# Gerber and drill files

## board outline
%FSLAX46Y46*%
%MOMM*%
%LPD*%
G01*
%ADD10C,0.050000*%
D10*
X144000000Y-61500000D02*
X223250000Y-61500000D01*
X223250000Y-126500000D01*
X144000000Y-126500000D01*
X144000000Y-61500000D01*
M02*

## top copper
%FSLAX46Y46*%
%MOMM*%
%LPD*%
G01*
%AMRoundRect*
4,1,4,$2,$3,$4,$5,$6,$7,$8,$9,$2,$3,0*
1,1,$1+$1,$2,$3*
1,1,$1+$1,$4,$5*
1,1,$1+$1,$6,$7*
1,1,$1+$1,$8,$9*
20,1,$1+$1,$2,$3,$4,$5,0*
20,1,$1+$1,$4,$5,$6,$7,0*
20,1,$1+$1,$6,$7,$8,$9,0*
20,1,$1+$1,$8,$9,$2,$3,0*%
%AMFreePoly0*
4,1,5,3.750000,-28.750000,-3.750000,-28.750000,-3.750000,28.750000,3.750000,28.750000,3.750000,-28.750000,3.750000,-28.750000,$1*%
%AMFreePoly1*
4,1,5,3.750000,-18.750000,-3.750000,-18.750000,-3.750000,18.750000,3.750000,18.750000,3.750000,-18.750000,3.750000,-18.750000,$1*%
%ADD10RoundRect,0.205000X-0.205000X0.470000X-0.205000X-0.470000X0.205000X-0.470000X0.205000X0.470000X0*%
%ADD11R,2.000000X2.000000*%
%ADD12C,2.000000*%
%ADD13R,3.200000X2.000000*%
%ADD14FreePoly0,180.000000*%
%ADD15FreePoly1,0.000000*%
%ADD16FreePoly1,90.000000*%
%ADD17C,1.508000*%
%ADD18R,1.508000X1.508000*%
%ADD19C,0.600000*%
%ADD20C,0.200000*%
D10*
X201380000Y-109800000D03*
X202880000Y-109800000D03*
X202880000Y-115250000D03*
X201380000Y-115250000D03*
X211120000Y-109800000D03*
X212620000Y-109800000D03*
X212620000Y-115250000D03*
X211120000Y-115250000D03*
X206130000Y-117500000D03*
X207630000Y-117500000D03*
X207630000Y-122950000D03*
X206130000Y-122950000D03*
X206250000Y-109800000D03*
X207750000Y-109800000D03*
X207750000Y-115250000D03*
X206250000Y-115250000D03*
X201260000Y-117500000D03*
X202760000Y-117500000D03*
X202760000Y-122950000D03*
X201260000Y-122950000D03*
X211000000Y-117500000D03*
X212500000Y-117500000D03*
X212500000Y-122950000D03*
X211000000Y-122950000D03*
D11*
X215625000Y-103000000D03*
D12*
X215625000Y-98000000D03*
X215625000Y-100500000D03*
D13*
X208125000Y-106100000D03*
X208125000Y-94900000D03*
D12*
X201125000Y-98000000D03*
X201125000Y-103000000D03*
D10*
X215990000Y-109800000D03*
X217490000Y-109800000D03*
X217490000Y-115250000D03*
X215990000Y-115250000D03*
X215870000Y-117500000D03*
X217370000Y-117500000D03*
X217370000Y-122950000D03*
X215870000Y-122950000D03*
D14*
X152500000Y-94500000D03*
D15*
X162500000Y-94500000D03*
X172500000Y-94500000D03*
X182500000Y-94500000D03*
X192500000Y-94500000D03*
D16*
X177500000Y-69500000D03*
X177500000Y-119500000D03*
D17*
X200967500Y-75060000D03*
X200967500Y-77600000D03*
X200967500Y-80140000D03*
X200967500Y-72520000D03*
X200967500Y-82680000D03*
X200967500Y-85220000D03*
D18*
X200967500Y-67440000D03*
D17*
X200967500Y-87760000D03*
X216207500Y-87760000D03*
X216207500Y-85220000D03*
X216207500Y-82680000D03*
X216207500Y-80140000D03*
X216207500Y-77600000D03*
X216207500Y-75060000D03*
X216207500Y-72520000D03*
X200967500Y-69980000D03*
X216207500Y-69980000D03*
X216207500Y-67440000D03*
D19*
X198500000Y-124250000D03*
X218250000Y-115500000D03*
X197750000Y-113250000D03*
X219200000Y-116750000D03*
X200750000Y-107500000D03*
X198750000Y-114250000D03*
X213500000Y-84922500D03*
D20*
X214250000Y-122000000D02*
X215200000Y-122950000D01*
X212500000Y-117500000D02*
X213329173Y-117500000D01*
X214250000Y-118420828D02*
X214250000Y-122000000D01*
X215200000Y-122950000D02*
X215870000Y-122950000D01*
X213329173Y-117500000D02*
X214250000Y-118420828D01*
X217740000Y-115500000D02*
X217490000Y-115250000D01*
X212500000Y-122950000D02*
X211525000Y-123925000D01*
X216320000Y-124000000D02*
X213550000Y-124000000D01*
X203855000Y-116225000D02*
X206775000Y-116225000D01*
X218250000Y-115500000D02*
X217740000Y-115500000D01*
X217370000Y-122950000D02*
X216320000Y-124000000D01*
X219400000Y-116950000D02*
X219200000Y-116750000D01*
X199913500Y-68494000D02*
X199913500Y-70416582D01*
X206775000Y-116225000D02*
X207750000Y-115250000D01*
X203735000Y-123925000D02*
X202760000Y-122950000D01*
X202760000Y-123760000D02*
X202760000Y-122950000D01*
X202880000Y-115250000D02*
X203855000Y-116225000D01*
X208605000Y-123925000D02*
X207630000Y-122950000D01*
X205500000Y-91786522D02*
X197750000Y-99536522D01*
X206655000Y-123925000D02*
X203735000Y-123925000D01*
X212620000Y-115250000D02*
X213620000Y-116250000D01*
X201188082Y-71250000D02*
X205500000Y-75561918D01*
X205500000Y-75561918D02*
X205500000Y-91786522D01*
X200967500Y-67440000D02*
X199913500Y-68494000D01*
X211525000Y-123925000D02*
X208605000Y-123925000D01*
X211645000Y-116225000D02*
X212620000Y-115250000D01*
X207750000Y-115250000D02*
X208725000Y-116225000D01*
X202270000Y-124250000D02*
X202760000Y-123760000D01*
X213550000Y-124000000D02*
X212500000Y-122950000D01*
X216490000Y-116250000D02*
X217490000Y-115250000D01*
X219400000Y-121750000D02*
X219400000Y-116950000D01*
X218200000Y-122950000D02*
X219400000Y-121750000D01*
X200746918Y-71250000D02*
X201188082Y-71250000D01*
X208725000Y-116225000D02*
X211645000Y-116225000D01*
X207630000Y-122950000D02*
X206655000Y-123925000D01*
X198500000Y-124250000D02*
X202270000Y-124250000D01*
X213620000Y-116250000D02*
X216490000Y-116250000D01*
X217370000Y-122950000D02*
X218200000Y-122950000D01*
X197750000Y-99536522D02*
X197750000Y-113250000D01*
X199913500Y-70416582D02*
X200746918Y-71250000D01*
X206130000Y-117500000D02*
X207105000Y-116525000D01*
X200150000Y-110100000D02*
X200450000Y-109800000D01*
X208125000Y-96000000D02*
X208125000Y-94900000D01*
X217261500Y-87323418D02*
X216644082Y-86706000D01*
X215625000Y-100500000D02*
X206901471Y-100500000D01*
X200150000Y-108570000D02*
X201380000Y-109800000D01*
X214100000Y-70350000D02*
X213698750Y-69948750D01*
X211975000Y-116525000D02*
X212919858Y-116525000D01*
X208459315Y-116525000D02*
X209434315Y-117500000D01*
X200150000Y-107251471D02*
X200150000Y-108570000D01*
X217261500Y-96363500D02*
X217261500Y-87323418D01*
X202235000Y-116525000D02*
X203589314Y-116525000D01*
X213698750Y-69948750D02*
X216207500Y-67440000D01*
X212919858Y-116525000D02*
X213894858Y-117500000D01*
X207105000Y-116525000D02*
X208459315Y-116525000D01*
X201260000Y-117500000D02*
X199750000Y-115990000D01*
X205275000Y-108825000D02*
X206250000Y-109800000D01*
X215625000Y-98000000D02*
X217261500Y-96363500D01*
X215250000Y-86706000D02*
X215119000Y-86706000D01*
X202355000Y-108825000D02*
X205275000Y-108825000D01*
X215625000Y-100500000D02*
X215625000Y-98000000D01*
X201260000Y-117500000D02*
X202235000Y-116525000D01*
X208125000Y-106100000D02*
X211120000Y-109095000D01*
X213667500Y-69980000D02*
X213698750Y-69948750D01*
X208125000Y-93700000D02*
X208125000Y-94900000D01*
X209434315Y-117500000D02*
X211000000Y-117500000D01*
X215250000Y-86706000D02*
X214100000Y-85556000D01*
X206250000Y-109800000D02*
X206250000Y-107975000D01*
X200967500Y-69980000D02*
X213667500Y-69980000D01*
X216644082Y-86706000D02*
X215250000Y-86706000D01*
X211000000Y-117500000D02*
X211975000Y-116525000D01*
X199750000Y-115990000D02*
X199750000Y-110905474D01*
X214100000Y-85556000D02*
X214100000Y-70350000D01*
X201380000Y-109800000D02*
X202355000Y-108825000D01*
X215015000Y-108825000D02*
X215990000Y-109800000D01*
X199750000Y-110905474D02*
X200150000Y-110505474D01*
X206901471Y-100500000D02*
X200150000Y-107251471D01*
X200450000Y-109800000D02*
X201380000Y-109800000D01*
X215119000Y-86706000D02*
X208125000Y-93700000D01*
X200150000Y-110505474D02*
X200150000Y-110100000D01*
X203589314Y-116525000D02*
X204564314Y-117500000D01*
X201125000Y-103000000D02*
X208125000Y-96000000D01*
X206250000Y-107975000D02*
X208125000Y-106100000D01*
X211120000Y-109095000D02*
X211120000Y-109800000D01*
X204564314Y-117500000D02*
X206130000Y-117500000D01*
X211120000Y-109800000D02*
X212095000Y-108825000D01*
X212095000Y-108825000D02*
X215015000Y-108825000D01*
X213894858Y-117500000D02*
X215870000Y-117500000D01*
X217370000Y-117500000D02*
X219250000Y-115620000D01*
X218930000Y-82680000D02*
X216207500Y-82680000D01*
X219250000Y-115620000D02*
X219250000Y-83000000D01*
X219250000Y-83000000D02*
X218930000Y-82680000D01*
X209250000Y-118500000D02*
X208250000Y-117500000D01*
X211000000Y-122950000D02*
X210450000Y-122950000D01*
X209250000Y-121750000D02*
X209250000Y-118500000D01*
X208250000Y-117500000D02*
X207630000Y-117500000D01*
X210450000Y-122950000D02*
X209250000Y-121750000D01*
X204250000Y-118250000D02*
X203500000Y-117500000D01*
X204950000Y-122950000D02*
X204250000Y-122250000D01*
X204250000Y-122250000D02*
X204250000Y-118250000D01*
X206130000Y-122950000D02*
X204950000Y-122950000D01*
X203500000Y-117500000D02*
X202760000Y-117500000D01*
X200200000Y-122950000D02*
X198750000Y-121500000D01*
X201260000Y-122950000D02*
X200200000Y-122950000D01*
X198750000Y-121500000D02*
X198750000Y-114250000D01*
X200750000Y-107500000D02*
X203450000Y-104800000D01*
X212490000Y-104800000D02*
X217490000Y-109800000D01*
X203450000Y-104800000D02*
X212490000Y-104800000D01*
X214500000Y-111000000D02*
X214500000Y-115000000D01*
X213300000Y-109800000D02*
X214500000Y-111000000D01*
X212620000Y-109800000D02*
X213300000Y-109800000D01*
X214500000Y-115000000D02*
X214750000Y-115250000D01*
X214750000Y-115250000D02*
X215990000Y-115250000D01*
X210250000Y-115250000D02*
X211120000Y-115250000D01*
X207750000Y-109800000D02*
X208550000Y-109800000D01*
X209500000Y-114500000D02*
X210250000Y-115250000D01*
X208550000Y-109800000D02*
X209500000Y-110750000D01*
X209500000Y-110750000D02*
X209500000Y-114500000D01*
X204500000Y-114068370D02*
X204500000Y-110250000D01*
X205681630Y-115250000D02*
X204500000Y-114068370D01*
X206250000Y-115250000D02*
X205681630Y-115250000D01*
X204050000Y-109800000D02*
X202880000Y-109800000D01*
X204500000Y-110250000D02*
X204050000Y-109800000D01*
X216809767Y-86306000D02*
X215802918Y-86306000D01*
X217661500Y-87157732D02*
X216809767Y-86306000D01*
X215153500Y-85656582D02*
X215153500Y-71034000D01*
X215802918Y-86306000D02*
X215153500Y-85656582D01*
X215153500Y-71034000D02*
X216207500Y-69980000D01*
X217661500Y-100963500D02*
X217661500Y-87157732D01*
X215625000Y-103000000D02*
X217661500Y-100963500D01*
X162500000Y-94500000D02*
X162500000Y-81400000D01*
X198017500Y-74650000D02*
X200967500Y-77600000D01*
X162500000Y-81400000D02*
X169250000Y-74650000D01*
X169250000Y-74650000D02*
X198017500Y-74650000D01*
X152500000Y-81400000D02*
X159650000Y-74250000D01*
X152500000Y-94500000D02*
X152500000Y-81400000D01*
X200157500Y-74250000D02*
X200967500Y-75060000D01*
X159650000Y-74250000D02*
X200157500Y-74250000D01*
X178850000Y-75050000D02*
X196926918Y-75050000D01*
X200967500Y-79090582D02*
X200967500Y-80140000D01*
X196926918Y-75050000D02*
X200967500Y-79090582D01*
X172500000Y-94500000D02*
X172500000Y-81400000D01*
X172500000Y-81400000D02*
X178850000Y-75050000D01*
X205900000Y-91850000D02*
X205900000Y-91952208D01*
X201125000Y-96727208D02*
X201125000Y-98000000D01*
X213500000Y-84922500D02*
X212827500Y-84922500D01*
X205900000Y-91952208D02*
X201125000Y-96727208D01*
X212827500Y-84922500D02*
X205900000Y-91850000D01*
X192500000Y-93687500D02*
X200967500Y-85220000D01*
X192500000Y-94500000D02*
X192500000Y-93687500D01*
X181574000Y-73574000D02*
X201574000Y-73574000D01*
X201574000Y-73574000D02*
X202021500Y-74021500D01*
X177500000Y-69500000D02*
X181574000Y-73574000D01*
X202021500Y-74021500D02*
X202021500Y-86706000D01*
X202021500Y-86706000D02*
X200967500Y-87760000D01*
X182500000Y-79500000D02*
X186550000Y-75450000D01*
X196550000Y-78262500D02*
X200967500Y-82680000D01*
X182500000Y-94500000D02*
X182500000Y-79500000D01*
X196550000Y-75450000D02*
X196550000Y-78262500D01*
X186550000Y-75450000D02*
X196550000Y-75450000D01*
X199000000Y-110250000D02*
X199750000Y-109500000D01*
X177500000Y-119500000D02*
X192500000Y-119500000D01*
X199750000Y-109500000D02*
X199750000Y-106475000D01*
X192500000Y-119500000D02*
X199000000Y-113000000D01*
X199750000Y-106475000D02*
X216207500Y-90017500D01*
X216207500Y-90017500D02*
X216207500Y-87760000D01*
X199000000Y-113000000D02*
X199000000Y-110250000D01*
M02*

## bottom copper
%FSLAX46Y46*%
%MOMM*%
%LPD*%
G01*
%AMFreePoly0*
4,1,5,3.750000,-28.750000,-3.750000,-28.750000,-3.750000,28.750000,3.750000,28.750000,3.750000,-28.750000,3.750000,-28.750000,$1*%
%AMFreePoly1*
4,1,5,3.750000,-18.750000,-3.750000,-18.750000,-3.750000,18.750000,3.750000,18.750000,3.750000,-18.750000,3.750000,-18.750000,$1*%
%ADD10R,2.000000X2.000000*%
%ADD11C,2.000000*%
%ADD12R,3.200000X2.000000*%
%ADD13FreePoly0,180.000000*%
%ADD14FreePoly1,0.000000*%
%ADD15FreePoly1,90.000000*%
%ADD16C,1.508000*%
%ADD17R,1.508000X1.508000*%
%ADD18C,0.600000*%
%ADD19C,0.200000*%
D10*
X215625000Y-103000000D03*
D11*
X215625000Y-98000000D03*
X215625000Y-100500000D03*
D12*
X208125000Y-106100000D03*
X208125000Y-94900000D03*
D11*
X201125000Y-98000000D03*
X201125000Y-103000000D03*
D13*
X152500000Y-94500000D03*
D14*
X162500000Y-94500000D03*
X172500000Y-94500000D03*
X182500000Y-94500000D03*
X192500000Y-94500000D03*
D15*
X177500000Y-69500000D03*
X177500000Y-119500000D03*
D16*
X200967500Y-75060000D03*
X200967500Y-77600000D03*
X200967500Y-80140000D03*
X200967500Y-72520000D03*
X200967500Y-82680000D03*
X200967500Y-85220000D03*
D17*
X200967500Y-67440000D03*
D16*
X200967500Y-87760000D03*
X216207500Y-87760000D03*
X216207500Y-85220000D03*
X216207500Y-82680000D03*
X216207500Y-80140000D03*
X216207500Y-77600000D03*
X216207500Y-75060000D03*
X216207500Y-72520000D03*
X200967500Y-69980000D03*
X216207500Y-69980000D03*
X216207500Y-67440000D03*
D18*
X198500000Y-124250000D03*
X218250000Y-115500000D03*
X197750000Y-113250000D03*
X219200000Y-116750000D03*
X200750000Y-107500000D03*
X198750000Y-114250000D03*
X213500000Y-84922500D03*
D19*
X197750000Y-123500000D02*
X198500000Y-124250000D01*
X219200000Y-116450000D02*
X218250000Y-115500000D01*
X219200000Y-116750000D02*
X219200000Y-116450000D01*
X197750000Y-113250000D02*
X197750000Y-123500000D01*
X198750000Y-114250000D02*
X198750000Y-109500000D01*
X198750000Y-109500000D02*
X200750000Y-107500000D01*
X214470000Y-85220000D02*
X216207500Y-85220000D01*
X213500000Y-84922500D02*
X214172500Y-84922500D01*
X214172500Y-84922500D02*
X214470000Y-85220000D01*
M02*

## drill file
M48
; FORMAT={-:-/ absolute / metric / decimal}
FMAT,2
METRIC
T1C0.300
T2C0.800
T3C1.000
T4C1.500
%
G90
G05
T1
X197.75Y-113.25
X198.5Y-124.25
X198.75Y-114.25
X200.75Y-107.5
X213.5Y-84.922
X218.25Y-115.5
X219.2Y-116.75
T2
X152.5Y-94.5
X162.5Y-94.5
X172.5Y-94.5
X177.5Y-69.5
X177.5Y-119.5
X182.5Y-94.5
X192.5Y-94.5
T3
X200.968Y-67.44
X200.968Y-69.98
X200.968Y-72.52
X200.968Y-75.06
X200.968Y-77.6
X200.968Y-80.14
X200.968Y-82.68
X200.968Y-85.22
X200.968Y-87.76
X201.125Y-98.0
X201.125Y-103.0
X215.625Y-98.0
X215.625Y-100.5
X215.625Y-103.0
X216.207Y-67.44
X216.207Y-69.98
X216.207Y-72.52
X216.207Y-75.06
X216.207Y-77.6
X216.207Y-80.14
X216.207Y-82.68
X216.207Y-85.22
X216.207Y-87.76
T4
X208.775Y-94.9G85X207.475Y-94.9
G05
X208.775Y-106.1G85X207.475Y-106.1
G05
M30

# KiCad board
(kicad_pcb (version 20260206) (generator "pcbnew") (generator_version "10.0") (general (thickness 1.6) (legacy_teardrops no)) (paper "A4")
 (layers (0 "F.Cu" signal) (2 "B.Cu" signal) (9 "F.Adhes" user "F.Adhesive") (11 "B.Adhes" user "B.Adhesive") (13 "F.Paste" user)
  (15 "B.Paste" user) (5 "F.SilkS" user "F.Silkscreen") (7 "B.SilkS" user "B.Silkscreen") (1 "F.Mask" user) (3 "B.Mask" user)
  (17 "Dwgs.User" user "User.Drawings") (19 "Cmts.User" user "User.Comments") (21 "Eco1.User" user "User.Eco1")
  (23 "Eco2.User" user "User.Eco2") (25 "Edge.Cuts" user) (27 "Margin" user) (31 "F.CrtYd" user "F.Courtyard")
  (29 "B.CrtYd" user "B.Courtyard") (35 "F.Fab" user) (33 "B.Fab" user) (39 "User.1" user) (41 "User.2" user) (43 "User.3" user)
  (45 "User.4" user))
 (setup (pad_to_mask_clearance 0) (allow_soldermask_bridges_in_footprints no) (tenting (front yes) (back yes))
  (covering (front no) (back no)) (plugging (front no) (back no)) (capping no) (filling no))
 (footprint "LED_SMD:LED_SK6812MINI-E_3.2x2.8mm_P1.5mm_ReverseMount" (layer "F.Cu") (at 202.13 112.525 -90)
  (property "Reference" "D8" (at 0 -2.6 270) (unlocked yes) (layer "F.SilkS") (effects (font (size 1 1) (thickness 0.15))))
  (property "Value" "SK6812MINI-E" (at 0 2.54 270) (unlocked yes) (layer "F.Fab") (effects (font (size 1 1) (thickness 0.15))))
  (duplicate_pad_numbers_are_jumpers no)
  (pad "1" smd roundrect (at -2.725 0.75 270) (size 1.35 0.82) (layers "F.Cu" "F.Mask" "F.Paste") (roundrect_rratio 0.25) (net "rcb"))
  (pad "2" smd roundrect (at -2.725 -0.75 270) (size 1.35 0.82) (layers "F.Cu" "F.Mask" "F.Paste") (roundrect_rratio 0.25)
   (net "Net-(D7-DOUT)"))
  (pad "3" smd roundrect (at 2.725 -0.75 270) (size 1.35 0.82) (layers "F.Cu" "F.Mask" "F.Paste") (roundrect_rratio 0.25) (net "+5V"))
  (pad "4" smd roundrect (at 2.725 0.75 270) (size 1.35 0.82) (layers "F.Cu" "F.Mask" "F.Paste") (roundrect_rratio 0.25)
   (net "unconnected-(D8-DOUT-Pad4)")))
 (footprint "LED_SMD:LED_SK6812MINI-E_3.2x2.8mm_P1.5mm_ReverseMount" (layer "F.Cu") (at 211.87 112.525 -90)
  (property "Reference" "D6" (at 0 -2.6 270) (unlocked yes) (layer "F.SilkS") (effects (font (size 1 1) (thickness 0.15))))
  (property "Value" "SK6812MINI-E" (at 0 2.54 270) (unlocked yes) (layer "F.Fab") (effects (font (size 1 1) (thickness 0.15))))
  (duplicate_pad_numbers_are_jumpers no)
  (pad "1" smd roundrect (at -2.725 0.75 270) (size 1.35 0.82) (layers "F.Cu" "F.Mask" "F.Paste") (roundrect_rratio 0.25) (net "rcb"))
  (pad "2" smd roundrect (at -2.725 -0.75 270) (size 1.35 0.82) (layers "F.Cu" "F.Mask" "F.Paste") (roundrect_rratio 0.25)
   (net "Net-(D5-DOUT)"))
  (pad "3" smd roundrect (at 2.725 -0.75 270) (size 1.35 0.82) (layers "F.Cu" "F.Mask" "F.Paste") (roundrect_rratio 0.25) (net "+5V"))
  (pad "4" smd roundrect (at 2.725 0.75 270) (size 1.35 0.82) (layers "F.Cu" "F.Mask" "F.Paste") (roundrect_rratio 0.25)
   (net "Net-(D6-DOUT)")))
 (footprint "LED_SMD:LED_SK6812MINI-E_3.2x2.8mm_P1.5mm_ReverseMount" (layer "F.Cu") (at 206.88 120.225 -90)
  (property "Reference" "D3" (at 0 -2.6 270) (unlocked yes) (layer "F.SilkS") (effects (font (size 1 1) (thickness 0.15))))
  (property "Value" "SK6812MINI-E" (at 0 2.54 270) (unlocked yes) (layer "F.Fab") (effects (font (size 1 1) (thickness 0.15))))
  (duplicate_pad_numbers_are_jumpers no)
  (pad "1" smd roundrect (at -2.725 0.75 270) (size 1.35 0.82) (layers "F.Cu" "F.Mask" "F.Paste") (roundrect_rratio 0.25) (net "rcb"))
  (pad "2" smd roundrect (at -2.725 -0.75 270) (size 1.35 0.82) (layers "F.Cu" "F.Mask" "F.Paste") (roundrect_rratio 0.25)
   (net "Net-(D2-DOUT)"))
  (pad "3" smd roundrect (at 2.725 -0.75 270) (size 1.35 0.82) (layers "F.Cu" "F.Mask" "F.Paste") (roundrect_rratio 0.25) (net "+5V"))
  (pad "4" smd roundrect (at 2.725 0.75 270) (size 1.35 0.82) (layers "F.Cu" "F.Mask" "F.Paste") (roundrect_rratio 0.25)
   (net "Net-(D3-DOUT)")))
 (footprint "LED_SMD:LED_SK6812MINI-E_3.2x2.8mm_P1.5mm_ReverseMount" (layer "F.Cu") (at 207 112.525 -90)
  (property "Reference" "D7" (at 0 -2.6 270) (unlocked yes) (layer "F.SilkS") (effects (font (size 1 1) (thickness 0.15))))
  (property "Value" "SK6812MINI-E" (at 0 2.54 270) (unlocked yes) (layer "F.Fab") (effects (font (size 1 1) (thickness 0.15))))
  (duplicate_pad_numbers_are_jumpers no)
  (pad "1" smd roundrect (at -2.725 0.75 270) (size 1.35 0.82) (layers "F.Cu" "F.Mask" "F.Paste") (roundrect_rratio 0.25) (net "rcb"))
  (pad "2" smd roundrect (at -2.725 -0.75 270) (size 1.35 0.82) (layers "F.Cu" "F.Mask" "F.Paste") (roundrect_rratio 0.25)
   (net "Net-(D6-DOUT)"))
  (pad "3" smd roundrect (at 2.725 -0.75 270) (size 1.35 0.82) (layers "F.Cu" "F.Mask" "F.Paste") (roundrect_rratio 0.25) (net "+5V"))
  (pad "4" smd roundrect (at 2.725 0.75 270) (size 1.35 0.82) (layers "F.Cu" "F.Mask" "F.Paste") (roundrect_rratio 0.25)
   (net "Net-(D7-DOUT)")))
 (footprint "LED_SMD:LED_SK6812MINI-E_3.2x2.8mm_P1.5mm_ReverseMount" (layer "F.Cu") (at 202.01 120.225 -90)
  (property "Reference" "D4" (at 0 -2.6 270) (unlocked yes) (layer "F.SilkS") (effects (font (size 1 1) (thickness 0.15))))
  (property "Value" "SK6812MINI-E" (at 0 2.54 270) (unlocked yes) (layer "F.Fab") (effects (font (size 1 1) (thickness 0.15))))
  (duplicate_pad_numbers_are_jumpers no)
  (pad "1" smd roundrect (at -2.725 0.75 270) (size 1.35 0.82) (layers "F.Cu" "F.Mask" "F.Paste") (roundrect_rratio 0.25) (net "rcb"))
  (pad "2" smd roundrect (at -2.725 -0.75 270) (size 1.35 0.82) (layers "F.Cu" "F.Mask" "F.Paste") (roundrect_rratio 0.25)
   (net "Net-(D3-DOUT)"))
  (pad "3" smd roundrect (at 2.725 -0.75 270) (size 1.35 0.82) (layers "F.Cu" "F.Mask" "F.Paste") (roundrect_rratio 0.25) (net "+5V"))
  (pad "4" smd roundrect (at 2.725 0.75 270) (size 1.35 0.82) (layers "F.Cu" "F.Mask" "F.Paste") (roundrect_rratio 0.25)
   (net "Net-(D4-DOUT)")))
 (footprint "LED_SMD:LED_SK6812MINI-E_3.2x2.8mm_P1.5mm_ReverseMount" (layer "F.Cu") (at 211.75 120.225 -90)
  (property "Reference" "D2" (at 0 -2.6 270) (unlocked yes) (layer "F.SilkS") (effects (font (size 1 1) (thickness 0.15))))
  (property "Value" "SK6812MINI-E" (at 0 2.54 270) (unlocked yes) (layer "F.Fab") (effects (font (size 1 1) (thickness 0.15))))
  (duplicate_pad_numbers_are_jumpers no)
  (pad "1" smd roundrect (at -2.725 0.75 270) (size 1.35 0.82) (layers "F.Cu" "F.Mask" "F.Paste") (roundrect_rratio 0.25) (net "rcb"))
  (pad "2" smd roundrect (at -2.725 -0.75 270) (size 1.35 0.82) (layers "F.Cu" "F.Mask" "F.Paste") (roundrect_rratio 0.25)
   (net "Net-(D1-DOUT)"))
  (pad "3" smd roundrect (at 2.725 -0.75 270) (size 1.35 0.82) (layers "F.Cu" "F.Mask" "F.Paste") (roundrect_rratio 0.25) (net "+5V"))
  (pad "4" smd roundrect (at 2.725 0.75 270) (size 1.35 0.82) (layers "F.Cu" "F.Mask" "F.Paste") (roundrect_rratio 0.25)
   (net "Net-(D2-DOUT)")))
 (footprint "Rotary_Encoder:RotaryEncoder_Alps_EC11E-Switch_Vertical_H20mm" (layer "F.Cu") (at 215.625 103 180)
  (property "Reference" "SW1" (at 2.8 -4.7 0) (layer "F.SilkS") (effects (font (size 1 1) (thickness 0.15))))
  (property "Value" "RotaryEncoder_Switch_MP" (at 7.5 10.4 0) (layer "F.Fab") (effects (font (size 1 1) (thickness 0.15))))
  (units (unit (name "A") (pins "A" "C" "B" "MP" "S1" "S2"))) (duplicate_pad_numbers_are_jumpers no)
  (pad "A" thru_hole rect (at 0 0 180) (size 2 2) (drill 1) (layers "*.Cu" "*.Mask") (remove_unused_layers no) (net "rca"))
  (pad "B" thru_hole circle (at 0 5 180) (size 2 2) (drill 1) (layers "*.Cu" "*.Mask") (remove_unused_layers no) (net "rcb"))
  (pad "C" thru_hole circle (at 0 2.5 180) (size 2 2) (drill 1) (layers "*.Cu" "*.Mask") (remove_unused_layers no) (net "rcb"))
  (pad "MP" thru_hole rect (at 7.5 -3.1 180) (size 3.2 2) (drill oval 2.8 1.5) (layers "*.Cu" "*.Mask") (remove_unused_layers no)
   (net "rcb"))
  (pad "MP" thru_hole rect (at 7.5 8.1 180) (size 3.2 2) (drill oval 2.8 1.5) (layers "*.Cu" "*.Mask") (remove_unused_layers no) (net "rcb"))
  (pad "S1" thru_hole circle (at 14.5 5 180) (size 2 2) (drill 1) (layers "*.Cu" "*.Mask") (remove_unused_layers no) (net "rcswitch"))
  (pad "S2" thru_hole circle (at 14.5 0 180) (size 2 2) (drill 1) (layers "*.Cu" "*.Mask") (remove_unused_layers no) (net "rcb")))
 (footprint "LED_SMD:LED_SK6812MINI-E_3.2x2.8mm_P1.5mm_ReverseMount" (layer "F.Cu") (at 216.74 112.525 -90)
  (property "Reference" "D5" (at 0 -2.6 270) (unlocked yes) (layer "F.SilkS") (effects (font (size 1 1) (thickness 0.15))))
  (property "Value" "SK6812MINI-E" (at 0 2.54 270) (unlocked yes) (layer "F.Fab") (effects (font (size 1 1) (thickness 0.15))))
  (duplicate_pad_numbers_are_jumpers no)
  (pad "1" smd roundrect (at -2.725 0.75 270) (size 1.35 0.82) (layers "F.Cu" "F.Mask" "F.Paste") (roundrect_rratio 0.25) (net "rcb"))
  (pad "2" smd roundrect (at -2.725 -0.75 270) (size 1.35 0.82) (layers "F.Cu" "F.Mask" "F.Paste") (roundrect_rratio 0.25)
   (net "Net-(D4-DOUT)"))
  (pad "3" smd roundrect (at 2.725 -0.75 270) (size 1.35 0.82) (layers "F.Cu" "F.Mask" "F.Paste") (roundrect_rratio 0.25) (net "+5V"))
  (pad "4" smd roundrect (at 2.725 0.75 270) (size 1.35 0.82) (layers "F.Cu" "F.Mask" "F.Paste") (roundrect_rratio 0.25)
   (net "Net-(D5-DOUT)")))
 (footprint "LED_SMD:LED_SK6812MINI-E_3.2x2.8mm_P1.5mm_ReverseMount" (layer "F.Cu") (at 216.62 120.225 -90)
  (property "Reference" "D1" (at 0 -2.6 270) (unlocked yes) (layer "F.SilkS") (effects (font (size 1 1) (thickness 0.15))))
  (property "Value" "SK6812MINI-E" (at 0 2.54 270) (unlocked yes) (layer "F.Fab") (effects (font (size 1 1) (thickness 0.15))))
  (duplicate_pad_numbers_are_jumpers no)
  (pad "1" smd roundrect (at -2.725 0.75 270) (size 1.35 0.82) (layers "F.Cu" "F.Mask" "F.Paste") (roundrect_rratio 0.25) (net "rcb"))
  (pad "2" smd roundrect (at -2.725 -0.75 270) (size 1.35 0.82) (layers "F.Cu" "F.Mask" "F.Paste") (roundrect_rratio 0.25) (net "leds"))
  (pad "3" smd roundrect (at 2.725 -0.75 270) (size 1.35 0.82) (layers "F.Cu" "F.Mask" "F.Paste") (roundrect_rratio 0.25) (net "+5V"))
  (pad "4" smd roundrect (at 2.725 0.75 270) (size 1.35 0.82) (layers "F.Cu" "F.Mask" "F.Paste") (roundrect_rratio 0.25)
   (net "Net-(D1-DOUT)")))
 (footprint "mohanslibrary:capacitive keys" (layer "F.Cu") (at 179.5 94.5 -90)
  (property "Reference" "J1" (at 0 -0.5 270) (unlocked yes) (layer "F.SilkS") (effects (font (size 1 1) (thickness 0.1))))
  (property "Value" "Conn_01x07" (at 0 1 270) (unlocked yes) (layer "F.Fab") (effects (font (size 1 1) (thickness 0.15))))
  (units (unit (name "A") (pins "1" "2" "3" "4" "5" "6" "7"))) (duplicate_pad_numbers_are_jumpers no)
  (pad "1" thru_hole custom (at 0 27 180) (size 7.5 57.5) (drill 0.8) (layers "*.Cu" "*.Mask") (remove_unused_layers no) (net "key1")
   (options (clearance outline) (anchor rect)) (primitives))
  (pad "2" thru_hole custom (at 0 17) (size 7.5 37.5) (drill 0.8) (layers "*.Cu" "*.Mask") (remove_unused_layers no) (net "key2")
   (options (clearance outline) (anchor rect)) (primitives))
  (pad "3" thru_hole custom (at 0 7) (size 7.5 37.5) (drill 0.8) (layers "*.Cu" "*.Mask") (remove_unused_layers no) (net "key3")
   (options (clearance outline) (anchor rect)) (primitives))
  (pad "4" thru_hole custom (at 0 -3) (size 7.5 37.5) (drill 0.8) (layers "*.Cu" "*.Mask") (remove_unused_layers no) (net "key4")
   (options (clearance outline) (anchor rect)) (primitives))
  (pad "5" thru_hole custom (at 0 -13) (size 7.5 37.5) (drill 0.8) (layers "*.Cu" "*.Mask") (remove_unused_layers no) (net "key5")
   (options (clearance outline) (anchor rect)) (primitives))
  (pad "6" thru_hole custom (at -25 2 90) (size 7.5 37.5) (drill 0.8) (layers "*.Cu" "*.Mask") (remove_unused_layers no) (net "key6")
   (options (clearance outline) (anchor rect)) (primitives))
  (pad "7" thru_hole custom (at 25 2 90) (size 7.5 37.5) (drill 0.8) (layers "*.Cu" "*.Mask") (remove_unused_layers no) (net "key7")
   (options (clearance outline) (anchor rect)) (primitives)))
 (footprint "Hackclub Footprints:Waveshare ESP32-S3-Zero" (layer "F.Cu") (at 208.5875 77.6)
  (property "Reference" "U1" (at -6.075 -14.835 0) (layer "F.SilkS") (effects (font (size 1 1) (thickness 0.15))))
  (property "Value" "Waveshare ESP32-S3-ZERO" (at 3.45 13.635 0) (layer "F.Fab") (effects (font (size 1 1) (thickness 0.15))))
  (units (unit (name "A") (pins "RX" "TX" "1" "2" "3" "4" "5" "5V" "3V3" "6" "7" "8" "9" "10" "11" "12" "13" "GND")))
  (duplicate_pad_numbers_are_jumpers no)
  (pad "1" thru_hole circle (at -7.62 -2.54) (size 1.508 1.508) (drill 1) (layers "*.Cu" "*.Mask") (remove_unused_layers no) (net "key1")
   (solder_mask_margin 0.102))
  (pad "2" thru_hole circle (at -7.62 0) (size 1.508 1.508) (drill 1) (layers "*.Cu" "*.Mask") (remove_unused_layers no) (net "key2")
   (solder_mask_margin 0.102))
  (pad "3" thru_hole circle (at -7.62 2.54) (size 1.508 1.508) (drill 1) (layers "*.Cu" "*.Mask") (remove_unused_layers no) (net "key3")
   (solder_mask_margin 0.102))
  (pad "3V3" thru_hole circle (at -7.62 -5.08) (size 1.508 1.508) (drill 1) (layers "*.Cu" "*.Mask") (remove_unused_layers no) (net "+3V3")
   (solder_mask_margin 0.102))
  (pad "4" thru_hole circle (at -7.62 5.08) (size 1.508 1.508) (drill 1) (layers "*.Cu" "*.Mask") (remove_unused_layers no) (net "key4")
   (solder_mask_margin 0.102))
  (pad "5" thru_hole circle (at -7.62 7.62) (size 1.508 1.508) (drill 1) (layers "*.Cu" "*.Mask") (remove_unused_layers no) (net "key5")
   (solder_mask_margin 0.102))
  (pad "5V" thru_hole rect (at -7.62 -10.16) (size 1.508 1.508) (drill 1) (layers "*.Cu" "*.Mask") (remove_unused_layers no) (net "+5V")
   (solder_mask_margin 0.102))
  (pad "6" thru_hole circle (at -7.62 10.16) (size 1.508 1.508) (drill 1) (layers "*.Cu" "*.Mask") (remove_unused_layers no) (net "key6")
   (solder_mask_margin 0.102))
  (pad "7" thru_hole circle (at 7.62 10.16) (size 1.508 1.508) (drill 1) (layers "*.Cu" "*.Mask") (remove_unused_layers no) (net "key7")
   (solder_mask_margin 0.102))
  (pad "8" thru_hole circle (at 7.62 7.62) (size 1.508 1.508) (drill 1) (layers "*.Cu" "*.Mask") (remove_unused_layers no) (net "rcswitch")
   (solder_mask_margin 0.102))
  (pad "9" thru_hole circle (at 7.62 5.08) (size 1.508 1.508) (drill 1) (layers "*.Cu" "*.Mask") (remove_unused_layers no) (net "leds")
   (solder_mask_margin 0.102))
  (pad "10" thru_hole circle (at 7.62 2.54) (size 1.508 1.508) (drill 1) (layers "*.Cu" "*.Mask") (remove_unused_layers no)
   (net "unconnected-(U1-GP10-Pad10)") (solder_mask_margin 0.102))
  (pad "11" thru_hole circle (at 7.62 0) (size 1.508 1.508) (drill 1) (layers "*.Cu" "*.Mask") (remove_unused_layers no)
   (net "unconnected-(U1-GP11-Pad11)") (solder_mask_margin 0.102))
  (pad "12" thru_hole circle (at 7.62 -2.54) (size 1.508 1.508) (drill 1) (layers "*.Cu" "*.Mask") (remove_unused_layers no)
   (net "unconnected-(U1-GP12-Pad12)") (solder_mask_margin 0.102))
  (pad "13" thru_hole circle (at 7.62 -5.08) (size 1.508 1.508) (drill 1) (layers "*.Cu" "*.Mask") (remove_unused_layers no)
   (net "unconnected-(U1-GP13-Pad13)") (solder_mask_margin 0.102))
  (pad "GND" thru_hole circle (at -7.62 -7.62) (size 1.508 1.508) (drill 1) (layers "*.Cu" "*.Mask") (remove_unused_layers no) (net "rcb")
   (solder_mask_margin 0.102))
  (pad "RX" thru_hole circle (at 7.62 -7.62) (size 1.508 1.508) (drill 1) (layers "*.Cu" "*.Mask") (remove_unused_layers no) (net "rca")
   (solder_mask_margin 0.102))
  (pad "TX" thru_hole circle (at 7.62 -10.16) (size 1.508 1.508) (drill 1) (layers "*.Cu" "*.Mask") (remove_unused_layers no) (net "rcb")
   (solder_mask_margin 0.102)))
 (gr_rect (start 144 61.5) (end 223.25 126.5) (stroke (width 0.05) (type default)) (fill no) (layer "Edge.Cuts"))
 (segment (start 214.25 122) (end 215.2 122.95) (width 0.2) (layer "F.Cu") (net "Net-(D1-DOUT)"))
 (segment (start 212.5 117.5) (end 213.329173 117.5) (width 0.2) (layer "F.Cu") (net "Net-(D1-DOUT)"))
 (segment (start 214.25 118.420828) (end 214.25 122) (width 0.2) (layer "F.Cu") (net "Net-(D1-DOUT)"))
 (segment (start 215.2 122.95) (end 215.87 122.95) (width 0.2) (layer "F.Cu") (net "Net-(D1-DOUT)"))
 (segment (start 213.329173 117.5) (end 214.25 118.420828) (width 0.2) (layer "F.Cu") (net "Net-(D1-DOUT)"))
 (segment (start 217.74 115.5) (end 217.49 115.25) (width 0.2) (layer "F.Cu") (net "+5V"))
 (segment (start 212.5 122.95) (end 211.525 123.925) (width 0.2) (layer "F.Cu") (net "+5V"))
 (segment (start 216.32 124) (end 213.55 124) (width 0.2) (layer "F.Cu") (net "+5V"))
 (segment (start 203.855 116.225) (end 206.775 116.225) (width 0.2) (layer "F.Cu") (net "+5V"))
 (segment (start 218.25 115.5) (end 217.74 115.5) (width 0.2) (layer "F.Cu") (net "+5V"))
 (segment (start 217.37 122.95) (end 216.32 124) (width 0.2) (layer "F.Cu") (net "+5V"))
 (segment (start 219.4 116.95) (end 219.2 116.75) (width 0.2) (layer "F.Cu") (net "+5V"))
 (segment (start 199.9135 68.494) (end 199.9135 70.416582) (width 0.2) (layer "F.Cu") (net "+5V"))
 (segment (start 206.775 116.225) (end 207.75 115.25) (width 0.2) (layer "F.Cu") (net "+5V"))
 (segment (start 203.735 123.925) (end 202.76 122.95) (width 0.2) (layer "F.Cu") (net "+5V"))
 (segment (start 202.76 123.76) (end 202.76 122.95) (width 0.2) (layer "F.Cu") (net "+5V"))
 (segment (start 202.88 115.25) (end 203.855 116.225) (width 0.2) (layer "F.Cu") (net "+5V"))
 (segment (start 208.605 123.925) (end 207.63 122.95) (width 0.2) (layer "F.Cu") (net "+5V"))
 (segment (start 205.5 91.786522) (end 197.75 99.536522) (width 0.2) (layer "F.Cu") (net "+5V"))
 (segment (start 206.655 123.925) (end 203.735 123.925) (width 0.2) (layer "F.Cu") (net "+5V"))
 (segment (start 212.62 115.25) (end 213.62 116.25) (width 0.2) (layer "F.Cu") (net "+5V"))
 (segment (start 201.188082 71.25) (end 205.5 75.561918) (width 0.2) (layer "F.Cu") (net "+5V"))
 (segment (start 205.5 75.561918) (end 205.5 91.786522) (width 0.2) (layer "F.Cu") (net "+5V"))
 (segment (start 200.9675 67.44) (end 199.9135 68.494) (width 0.2) (layer "F.Cu") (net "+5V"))
 (segment (start 211.525 123.925) (end 208.605 123.925) (width 0.2) (layer "F.Cu") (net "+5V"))
 (segment (start 211.645 116.225) (end 212.62 115.25) (width 0.2) (layer "F.Cu") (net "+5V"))
 (segment (start 207.75 115.25) (end 208.725 116.225) (width 0.2) (layer "F.Cu") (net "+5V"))
 (segment (start 202.27 124.25) (end 202.76 123.76) (width 0.2) (layer "F.Cu") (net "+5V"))
 (segment (start 213.55 124) (end 212.5 122.95) (width 0.2) (layer "F.Cu") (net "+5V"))
 (segment (start 216.49 116.25) (end 217.49 115.25) (width 0.2) (layer "F.Cu") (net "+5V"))
 (segment (start 219.4 121.75) (end 219.4 116.95) (width 0.2) (layer "F.Cu") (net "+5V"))
 (segment (start 218.2 122.95) (end 219.4 121.75) (width 0.2) (layer "F.Cu") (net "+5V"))
 (segment (start 200.746918 71.25) (end 201.188082 71.25) (width 0.2) (layer "F.Cu") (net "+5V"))
 (segment (start 208.725 116.225) (end 211.645 116.225) (width 0.2) (layer "F.Cu") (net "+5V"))
 (segment (start 207.63 122.95) (end 206.655 123.925) (width 0.2) (layer "F.Cu") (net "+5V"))
 (segment (start 198.5 124.25) (end 202.27 124.25) (width 0.2) (layer "F.Cu") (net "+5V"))
 (segment (start 213.62 116.25) (end 216.49 116.25) (width 0.2) (layer "F.Cu") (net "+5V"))
 (segment (start 217.37 122.95) (end 218.2 122.95) (width 0.2) (layer "F.Cu") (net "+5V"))
 (segment (start 197.75 99.536522) (end 197.75 113.25) (width 0.2) (layer "F.Cu") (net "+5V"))
 (segment (start 199.9135 70.416582) (end 200.746918 71.25) (width 0.2) (layer "F.Cu") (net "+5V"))
 (via (at 198.5 124.25) (size 0.6) (drill 0.3) (layers "F.Cu" "B.Cu") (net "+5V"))
 (via (at 218.25 115.5) (size 0.6) (drill 0.3) (layers "F.Cu" "B.Cu") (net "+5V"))
 (via (at 197.75 113.25) (size 0.6) (drill 0.3) (layers "F.Cu" "B.Cu") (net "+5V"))
 (via (at 219.2 116.75) (size 0.6) (drill 0.3) (layers "F.Cu" "B.Cu") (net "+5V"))
 (segment (start 197.75 123.5) (end 198.5 124.25) (width 0.2) (layer "B.Cu") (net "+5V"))
 (segment (start 219.2 116.45) (end 218.25 115.5) (width 0.2) (layer "B.Cu") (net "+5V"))
 (segment (start 219.2 116.75) (end 219.2 116.45) (width 0.2) (layer "B.Cu") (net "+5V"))
 (segment (start 197.75 113.25) (end 197.75 123.5) (width 0.2) (layer "B.Cu") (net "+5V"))
 (segment (start 206.13 117.5) (end 207.105 116.525) (width 0.2) (layer "F.Cu") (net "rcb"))
 (segment (start 200.15 110.1) (end 200.45 109.8) (width 0.2) (layer "F.Cu") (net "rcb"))
 (segment (start 208.125 96) (end 208.125 94.9) (width 0.2) (layer "F.Cu") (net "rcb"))
 (segment (start 217.2615 87.323418) (end 216.644082 86.706) (width 0.2) (layer "F.Cu") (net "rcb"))
 (segment (start 215.625 100.5) (end 206.901471 100.5) (width 0.2) (layer "F.Cu") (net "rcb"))
 (segment (start 200.15 108.57) (end 201.38 109.8) (width 0.2) (layer "F.Cu") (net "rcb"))
 (segment (start 214.1 70.35) (end 213.69875 69.94875) (width 0.2) (layer "F.Cu") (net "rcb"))
 (segment (start 211.975 116.525) (end 212.919858 116.525) (width 0.2) (layer "F.Cu") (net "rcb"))
 (segment (start 208.459315 116.525) (end 209.434315 117.5) (width 0.2) (layer "F.Cu") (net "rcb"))
 (segment (start 200.15 107.251471) (end 200.15 108.57) (width 0.2) (layer "F.Cu") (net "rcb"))
 (segment (start 217.2615 96.3635) (end 217.2615 87.323418) (width 0.2) (layer "F.Cu") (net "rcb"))
 (segment (start 202.235 116.525) (end 203.589314 116.525) (width 0.2) (layer "F.Cu") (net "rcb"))
 (segment (start 213.69875 69.94875) (end 216.2075 67.44) (width 0.2) (layer "F.Cu") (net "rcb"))
 (segment (start 212.919858 116.525) (end 213.894858 117.5) (width 0.2) (layer "F.Cu") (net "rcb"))
 (segment (start 207.105 116.525) (end 208.459315 116.525) (width 0.2) (layer "F.Cu") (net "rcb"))
 (segment (start 201.26 117.5) (end 199.75 115.99) (width 0.2) (layer "F.Cu") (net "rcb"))
 (segment (start 205.275 108.825) (end 206.25 109.8) (width 0.2) (layer "F.Cu") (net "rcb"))
 (segment (start 215.625 98) (end 217.2615 96.3635) (width 0.2) (layer "F.Cu") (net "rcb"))
 (segment (start 215.25 86.706) (end 215.119 86.706) (width 0.2) (layer "F.Cu") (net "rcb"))
 (segment (start 202.355 108.825) (end 205.275 108.825) (width 0.2) (layer "F.Cu") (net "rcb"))
 (segment (start 215.625 100.5) (end 215.625 98) (width 0.2) (layer "F.Cu") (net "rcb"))
 (segment (start 201.26 117.5) (end 202.235 116.525) (width 0.2) (layer "F.Cu") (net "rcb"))
 (segment (start 208.125 106.1) (end 211.12 109.095) (width 0.2) (layer "F.Cu") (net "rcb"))
 (segment (start 213.6675 69.98) (end 213.69875 69.94875) (width 0.2) (layer "F.Cu") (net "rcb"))
 (segment (start 208.125 93.7) (end 208.125 94.9) (width 0.2) (layer "F.Cu") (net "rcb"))
 (segment (start 209.434315 117.5) (end 211 117.5) (width 0.2) (layer "F.Cu") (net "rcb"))
 (segment (start 215.25 86.706) (end 214.1 85.556) (width 0.2) (layer "F.Cu") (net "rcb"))
 (segment (start 206.25 109.8) (end 206.25 107.975) (width 0.2) (layer "F.Cu") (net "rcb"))
 (segment (start 200.9675 69.98) (end 213.6675 69.98) (width 0.2) (layer "F.Cu") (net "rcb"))
 (segment (start 216.644082 86.706) (end 215.25 86.706) (width 0.2) (layer "F.Cu") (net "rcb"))
 (segment (start 211 117.5) (end 211.975 116.525) (width 0.2) (layer "F.Cu") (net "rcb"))
 (segment (start 199.75 115.99) (end 199.75 110.905474) (width 0.2) (layer "F.Cu") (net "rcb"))
 (segment (start 214.1 85.556) (end 214.1 70.35) (width 0.2) (layer "F.Cu") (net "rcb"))
 (segment (start 201.38 109.8) (end 202.355 108.825) (width 0.2) (layer "F.Cu") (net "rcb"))
 (segment (start 215.015 108.825) (end 215.99 109.8) (width 0.2) (layer "F.Cu") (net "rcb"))
 (segment (start 199.75 110.905474) (end 200.15 110.505474) (width 0.2) (layer "F.Cu") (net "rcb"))
 (segment (start 206.901471 100.5) (end 200.15 107.251471) (width 0.2) (layer "F.Cu") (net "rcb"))
 (segment (start 200.45 109.8) (end 201.38 109.8) (width 0.2) (layer "F.Cu") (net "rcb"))
 (segment (start 215.119 86.706) (end 208.125 93.7) (width 0.2) (layer "F.Cu") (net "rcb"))
 (segment (start 200.15 110.505474) (end 200.15 110.1) (width 0.2) (layer "F.Cu") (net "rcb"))
 (segment (start 203.589314 116.525) (end 204.564314 117.5) (width 0.2) (layer "F.Cu") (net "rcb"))
 (segment (start 201.125 103) (end 208.125 96) (width 0.2) (layer "F.Cu") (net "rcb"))
 (segment (start 206.25 107.975) (end 208.125 106.1) (width 0.2) (layer "F.Cu") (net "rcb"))
 (segment (start 211.12 109.095) (end 211.12 109.8) (width 0.2) (layer "F.Cu") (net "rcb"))
 (segment (start 204.564314 117.5) (end 206.13 117.5) (width 0.2) (layer "F.Cu") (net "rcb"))
 (segment (start 211.12 109.8) (end 212.095 108.825) (width 0.2) (layer "F.Cu") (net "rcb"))
 (segment (start 212.095 108.825) (end 215.015 108.825) (width 0.2) (layer "F.Cu") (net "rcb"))
 (segment (start 213.894858 117.5) (end 215.87 117.5) (width 0.2) (layer "F.Cu") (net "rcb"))
 (segment (start 217.37 117.5) (end 219.25 115.62) (width 0.2) (layer "F.Cu") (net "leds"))
 (segment (start 218.93 82.68) (end 216.2075 82.68) (width 0.2) (layer "F.Cu") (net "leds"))
 (segment (start 219.25 115.62) (end 219.25 83) (width 0.2) (layer "F.Cu") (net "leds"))
 (segment (start 219.25 83) (end 218.93 82.68) (width 0.2) (layer "F.Cu") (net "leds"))
 (segment (start 209.25 118.5) (end 208.25 117.5) (width 0.2) (layer "F.Cu") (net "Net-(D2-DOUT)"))
 (segment (start 211 122.95) (end 210.45 122.95) (width 0.2) (layer "F.Cu") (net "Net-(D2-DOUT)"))
 (segment (start 209.25 121.75) (end 209.25 118.5) (width 0.2) (layer "F.Cu") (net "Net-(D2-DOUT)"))
 (segment (start 208.25 117.5) (end 207.63 117.5) (width 0.2) (layer "F.Cu") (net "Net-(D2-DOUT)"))
 (segment (start 210.45 122.95) (end 209.25 121.75) (width 0.2) (layer "F.Cu") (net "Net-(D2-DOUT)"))
 (segment (start 204.25 118.25) (end 203.5 117.5) (width 0.2) (layer "F.Cu") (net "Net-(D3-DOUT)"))
 (segment (start 204.95 122.95) (end 204.25 122.25) (width 0.2) (layer "F.Cu") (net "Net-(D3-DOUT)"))
 (segment (start 204.25 122.25) (end 204.25 118.25) (width 0.2) (layer "F.Cu") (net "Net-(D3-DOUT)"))
 (segment (start 206.13 122.95) (end 204.95 122.95) (width 0.2) (layer "F.Cu") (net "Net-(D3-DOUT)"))
 (segment (start 203.5 117.5) (end 202.76 117.5) (width 0.2) (layer "F.Cu") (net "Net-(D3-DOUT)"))
 (segment (start 200.2 122.95) (end 198.75 121.5) (width 0.2) (layer "F.Cu") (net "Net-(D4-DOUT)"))
 (segment (start 201.26 122.95) (end 200.2 122.95) (width 0.2) (layer "F.Cu") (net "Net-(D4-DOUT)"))
 (segment (start 198.75 121.5) (end 198.75 114.25) (width 0.2) (layer "F.Cu") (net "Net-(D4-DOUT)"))
 (segment (start 200.75 107.5) (end 203.45 104.8) (width 0.2) (layer "F.Cu") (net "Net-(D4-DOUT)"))
 (segment (start 212.49 104.8) (end 217.49 109.8) (width 0.2) (layer "F.Cu") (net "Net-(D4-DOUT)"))
 (segment (start 203.45 104.8) (end 212.49 104.8) (width 0.2) (layer "F.Cu") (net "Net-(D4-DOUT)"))
 (via (at 200.75 107.5) (size 0.6) (drill 0.3) (layers "F.Cu" "B.Cu") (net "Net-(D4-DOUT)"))
 (via (at 198.75 114.25) (size 0.6) (drill 0.3) (layers "F.Cu" "B.Cu") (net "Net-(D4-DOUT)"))
 (segment (start 198.75 114.25) (end 198.75 109.5) (width 0.2) (layer "B.Cu") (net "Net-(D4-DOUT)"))
 (segment (start 198.75 109.5) (end 200.75 107.5) (width 0.2) (layer "B.Cu") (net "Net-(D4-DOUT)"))
 (segment (start 214.5 111) (end 214.5 115) (width 0.2) (layer "F.Cu") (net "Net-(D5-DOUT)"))
 (segment (start 213.3 109.8) (end 214.5 111) (width 0.2) (layer "F.Cu") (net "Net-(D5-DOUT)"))
 (segment (start 212.62 109.8) (end 213.3 109.8) (width 0.2) (layer "F.Cu") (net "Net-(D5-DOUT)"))
 (segment (start 214.5 115) (end 214.75 115.25) (width 0.2) (layer "F.Cu") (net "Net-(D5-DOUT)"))
 (segment (start 214.75 115.25) (end 215.99 115.25) (width 0.2) (layer "F.Cu") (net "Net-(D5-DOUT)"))
 (segment (start 210.25 115.25) (end 211.12 115.25) (width 0.2) (layer "F.Cu") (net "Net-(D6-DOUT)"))
 (segment (start 207.75 109.8) (end 208.55 109.8) (width 0.2) (layer "F.Cu") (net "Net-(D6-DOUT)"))
 (segment (start 209.5 114.5) (end 210.25 115.25) (width 0.2) (layer "F.Cu") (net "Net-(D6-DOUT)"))
 (segment (start 208.55 109.8) (end 209.5 110.75) (width 0.2) (layer "F.Cu") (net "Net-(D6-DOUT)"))
 (segment (start 209.5 110.75) (end 209.5 114.5) (width 0.2) (layer "F.Cu") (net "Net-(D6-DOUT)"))
 (segment (start 204.5 114.06837) (end 204.5 110.25) (width 0.2) (layer "F.Cu") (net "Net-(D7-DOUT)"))
 (segment (start 205.68163 115.25) (end 204.5 114.06837) (width 0.2) (layer "F.Cu") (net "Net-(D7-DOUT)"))
 (segment (start 206.25 115.25) (end 205.68163 115.25) (width 0.2) (layer "F.Cu") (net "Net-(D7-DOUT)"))
 (segment (start 204.05 109.8) (end 202.88 109.8) (width 0.2) (layer "F.Cu") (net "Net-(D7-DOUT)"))
 (segment (start 204.5 110.25) (end 204.05 109.8) (width 0.2) (layer "F.Cu") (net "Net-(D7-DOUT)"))
 (segment (start 216.809767 86.306) (end 215.802918 86.306) (width 0.2) (layer "F.Cu") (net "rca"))
 (segment (start 217.6615 87.157732) (end 216.809767 86.306) (width 0.2) (layer "F.Cu") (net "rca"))
 (segment (start 215.1535 85.656582) (end 215.1535 71.034) (width 0.2) (layer "F.Cu") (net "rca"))
 (segment (start 215.802918 86.306) (end 215.1535 85.656582) (width 0.2) (layer "F.Cu") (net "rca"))
 (segment (start 215.1535 71.034) (end 216.2075 69.98) (width 0.2) (layer "F.Cu") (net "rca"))
 (segment (start 217.6615 100.9635) (end 217.6615 87.157732) (width 0.2) (layer "F.Cu") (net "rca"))
 (segment (start 215.625 103) (end 217.6615 100.9635) (width 0.2) (layer "F.Cu") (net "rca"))
 (segment (start 162.5 94.5) (end 162.5 81.4) (width 0.2) (layer "F.Cu") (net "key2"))
 (segment (start 198.0175 74.65) (end 200.9675 77.6) (width 0.2) (layer "F.Cu") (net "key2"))
 (segment (start 162.5 81.4) (end 169.25 74.65) (width 0.2) (layer "F.Cu") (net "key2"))
 (segment (start 169.25 74.65) (end 198.0175 74.65) (width 0.2) (layer "F.Cu") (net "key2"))
 (segment (start 152.5 81.4) (end 159.65 74.25) (width 0.2) (layer "F.Cu") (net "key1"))
 (segment (start 152.5 94.5) (end 152.5 81.4) (width 0.2) (layer "F.Cu") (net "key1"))
 (segment (start 200.1575 74.25) (end 200.9675 75.06) (width 0.2) (layer "F.Cu") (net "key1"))
 (segment (start 159.65 74.25) (end 200.1575 74.25) (width 0.2) (layer "F.Cu") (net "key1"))
 (segment (start 178.85 75.05) (end 196.926918 75.05) (width 0.2) (layer "F.Cu") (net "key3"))
 (segment (start 200.9675 79.090582) (end 200.9675 80.14) (width 0.2) (layer "F.Cu") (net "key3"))
 (segment (start 196.926918 75.05) (end 200.9675 79.090582) (width 0.2) (layer "F.Cu") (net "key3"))
 (segment (start 172.5 94.5) (end 172.5 81.4) (width 0.2) (layer "F.Cu") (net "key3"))
 (segment (start 172.5 81.4) (end 178.85 75.05) (width 0.2) (layer "F.Cu") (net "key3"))
 (segment (start 205.9 91.85) (end 205.9 91.952208) (width 0.2) (layer "F.Cu") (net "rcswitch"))
 (segment (start 201.125 96.727208) (end 201.125 98) (width 0.2) (layer "F.Cu") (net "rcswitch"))
 (segment (start 213.5 84.9225) (end 212.8275 84.9225) (width 0.2) (layer "F.Cu") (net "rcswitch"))
 (segment (start 205.9 91.952208) (end 201.125 96.727208) (width 0.2) (layer "F.Cu") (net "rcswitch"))
 (segment (start 212.8275 84.9225) (end 205.9 91.85) (width 0.2) (layer "F.Cu") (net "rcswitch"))
 (via (at 213.5 84.9225) (size 0.6) (drill 0.3) (layers "F.Cu" "B.Cu") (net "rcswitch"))
 (segment (start 214.47 85.22) (end 216.2075 85.22) (width 0.2) (layer "B.Cu") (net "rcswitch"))
 (segment (start 213.5 84.9225) (end 214.1725 84.9225) (width 0.2) (layer "B.Cu") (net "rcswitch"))
 (segment (start 214.1725 84.9225) (end 214.47 85.22) (width 0.2) (layer "B.Cu") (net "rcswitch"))
 (segment (start 192.5 93.6875) (end 200.9675 85.22) (width 0.2) (layer "F.Cu") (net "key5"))
 (segment (start 192.5 94.5) (end 192.5 93.6875) (width 0.2) (layer "F.Cu") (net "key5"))
 (segment (start 181.574 73.574) (end 201.574 73.574) (width 0.2) (layer "F.Cu") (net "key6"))
 (segment (start 201.574 73.574) (end 202.0215 74.0215) (width 0.2) (layer "F.Cu") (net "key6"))
 (segment (start 177.5 69.5) (end 181.574 73.574) (width 0.2) (layer "F.Cu") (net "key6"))
 (segment (start 202.0215 74.0215) (end 202.0215 86.706) (width 0.2) (layer "F.Cu") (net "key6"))
 (segment (start 202.0215 86.706) (end 200.9675 87.76) (width 0.2) (layer "F.Cu") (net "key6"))
 (segment (start 182.5 79.5) (end 186.55 75.45) (width 0.2) (layer "F.Cu") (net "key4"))
 (segment (start 196.55 78.2625) (end 200.9675 82.68) (width 0.2) (layer "F.Cu") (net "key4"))
 (segment (start 182.5 94.5) (end 182.5 79.5) (width 0.2) (layer "F.Cu") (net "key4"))
 (segment (start 196.55 75.45) (end 196.55 78.2625) (width 0.2) (layer "F.Cu") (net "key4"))
 (segment (start 186.55 75.45) (end 196.55 75.45) (width 0.2) (layer "F.Cu") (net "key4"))
 (segment (start 199 110.25) (end 199.75 109.5) (width 0.2) (layer "F.Cu") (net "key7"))
 (segment (start 177.5 119.5) (end 192.5 119.5) (width 0.2) (layer "F.Cu") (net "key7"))
 (segment (start 199.75 109.5) (end 199.75 106.475) (width 0.2) (layer "F.Cu") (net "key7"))
 (segment (start 192.5 119.5) (end 199 113) (width 0.2) (layer "F.Cu") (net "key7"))
 (segment (start 199.75 106.475) (end 216.2075 90.0175) (width 0.2) (layer "F.Cu") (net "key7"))
 (segment (start 216.2075 90.0175) (end 216.2075 87.76) (width 0.2) (layer "F.Cu") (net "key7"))
 (segment (start 199 113) (end 199 110.25) (width 0.2) (layer "F.Cu") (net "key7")))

